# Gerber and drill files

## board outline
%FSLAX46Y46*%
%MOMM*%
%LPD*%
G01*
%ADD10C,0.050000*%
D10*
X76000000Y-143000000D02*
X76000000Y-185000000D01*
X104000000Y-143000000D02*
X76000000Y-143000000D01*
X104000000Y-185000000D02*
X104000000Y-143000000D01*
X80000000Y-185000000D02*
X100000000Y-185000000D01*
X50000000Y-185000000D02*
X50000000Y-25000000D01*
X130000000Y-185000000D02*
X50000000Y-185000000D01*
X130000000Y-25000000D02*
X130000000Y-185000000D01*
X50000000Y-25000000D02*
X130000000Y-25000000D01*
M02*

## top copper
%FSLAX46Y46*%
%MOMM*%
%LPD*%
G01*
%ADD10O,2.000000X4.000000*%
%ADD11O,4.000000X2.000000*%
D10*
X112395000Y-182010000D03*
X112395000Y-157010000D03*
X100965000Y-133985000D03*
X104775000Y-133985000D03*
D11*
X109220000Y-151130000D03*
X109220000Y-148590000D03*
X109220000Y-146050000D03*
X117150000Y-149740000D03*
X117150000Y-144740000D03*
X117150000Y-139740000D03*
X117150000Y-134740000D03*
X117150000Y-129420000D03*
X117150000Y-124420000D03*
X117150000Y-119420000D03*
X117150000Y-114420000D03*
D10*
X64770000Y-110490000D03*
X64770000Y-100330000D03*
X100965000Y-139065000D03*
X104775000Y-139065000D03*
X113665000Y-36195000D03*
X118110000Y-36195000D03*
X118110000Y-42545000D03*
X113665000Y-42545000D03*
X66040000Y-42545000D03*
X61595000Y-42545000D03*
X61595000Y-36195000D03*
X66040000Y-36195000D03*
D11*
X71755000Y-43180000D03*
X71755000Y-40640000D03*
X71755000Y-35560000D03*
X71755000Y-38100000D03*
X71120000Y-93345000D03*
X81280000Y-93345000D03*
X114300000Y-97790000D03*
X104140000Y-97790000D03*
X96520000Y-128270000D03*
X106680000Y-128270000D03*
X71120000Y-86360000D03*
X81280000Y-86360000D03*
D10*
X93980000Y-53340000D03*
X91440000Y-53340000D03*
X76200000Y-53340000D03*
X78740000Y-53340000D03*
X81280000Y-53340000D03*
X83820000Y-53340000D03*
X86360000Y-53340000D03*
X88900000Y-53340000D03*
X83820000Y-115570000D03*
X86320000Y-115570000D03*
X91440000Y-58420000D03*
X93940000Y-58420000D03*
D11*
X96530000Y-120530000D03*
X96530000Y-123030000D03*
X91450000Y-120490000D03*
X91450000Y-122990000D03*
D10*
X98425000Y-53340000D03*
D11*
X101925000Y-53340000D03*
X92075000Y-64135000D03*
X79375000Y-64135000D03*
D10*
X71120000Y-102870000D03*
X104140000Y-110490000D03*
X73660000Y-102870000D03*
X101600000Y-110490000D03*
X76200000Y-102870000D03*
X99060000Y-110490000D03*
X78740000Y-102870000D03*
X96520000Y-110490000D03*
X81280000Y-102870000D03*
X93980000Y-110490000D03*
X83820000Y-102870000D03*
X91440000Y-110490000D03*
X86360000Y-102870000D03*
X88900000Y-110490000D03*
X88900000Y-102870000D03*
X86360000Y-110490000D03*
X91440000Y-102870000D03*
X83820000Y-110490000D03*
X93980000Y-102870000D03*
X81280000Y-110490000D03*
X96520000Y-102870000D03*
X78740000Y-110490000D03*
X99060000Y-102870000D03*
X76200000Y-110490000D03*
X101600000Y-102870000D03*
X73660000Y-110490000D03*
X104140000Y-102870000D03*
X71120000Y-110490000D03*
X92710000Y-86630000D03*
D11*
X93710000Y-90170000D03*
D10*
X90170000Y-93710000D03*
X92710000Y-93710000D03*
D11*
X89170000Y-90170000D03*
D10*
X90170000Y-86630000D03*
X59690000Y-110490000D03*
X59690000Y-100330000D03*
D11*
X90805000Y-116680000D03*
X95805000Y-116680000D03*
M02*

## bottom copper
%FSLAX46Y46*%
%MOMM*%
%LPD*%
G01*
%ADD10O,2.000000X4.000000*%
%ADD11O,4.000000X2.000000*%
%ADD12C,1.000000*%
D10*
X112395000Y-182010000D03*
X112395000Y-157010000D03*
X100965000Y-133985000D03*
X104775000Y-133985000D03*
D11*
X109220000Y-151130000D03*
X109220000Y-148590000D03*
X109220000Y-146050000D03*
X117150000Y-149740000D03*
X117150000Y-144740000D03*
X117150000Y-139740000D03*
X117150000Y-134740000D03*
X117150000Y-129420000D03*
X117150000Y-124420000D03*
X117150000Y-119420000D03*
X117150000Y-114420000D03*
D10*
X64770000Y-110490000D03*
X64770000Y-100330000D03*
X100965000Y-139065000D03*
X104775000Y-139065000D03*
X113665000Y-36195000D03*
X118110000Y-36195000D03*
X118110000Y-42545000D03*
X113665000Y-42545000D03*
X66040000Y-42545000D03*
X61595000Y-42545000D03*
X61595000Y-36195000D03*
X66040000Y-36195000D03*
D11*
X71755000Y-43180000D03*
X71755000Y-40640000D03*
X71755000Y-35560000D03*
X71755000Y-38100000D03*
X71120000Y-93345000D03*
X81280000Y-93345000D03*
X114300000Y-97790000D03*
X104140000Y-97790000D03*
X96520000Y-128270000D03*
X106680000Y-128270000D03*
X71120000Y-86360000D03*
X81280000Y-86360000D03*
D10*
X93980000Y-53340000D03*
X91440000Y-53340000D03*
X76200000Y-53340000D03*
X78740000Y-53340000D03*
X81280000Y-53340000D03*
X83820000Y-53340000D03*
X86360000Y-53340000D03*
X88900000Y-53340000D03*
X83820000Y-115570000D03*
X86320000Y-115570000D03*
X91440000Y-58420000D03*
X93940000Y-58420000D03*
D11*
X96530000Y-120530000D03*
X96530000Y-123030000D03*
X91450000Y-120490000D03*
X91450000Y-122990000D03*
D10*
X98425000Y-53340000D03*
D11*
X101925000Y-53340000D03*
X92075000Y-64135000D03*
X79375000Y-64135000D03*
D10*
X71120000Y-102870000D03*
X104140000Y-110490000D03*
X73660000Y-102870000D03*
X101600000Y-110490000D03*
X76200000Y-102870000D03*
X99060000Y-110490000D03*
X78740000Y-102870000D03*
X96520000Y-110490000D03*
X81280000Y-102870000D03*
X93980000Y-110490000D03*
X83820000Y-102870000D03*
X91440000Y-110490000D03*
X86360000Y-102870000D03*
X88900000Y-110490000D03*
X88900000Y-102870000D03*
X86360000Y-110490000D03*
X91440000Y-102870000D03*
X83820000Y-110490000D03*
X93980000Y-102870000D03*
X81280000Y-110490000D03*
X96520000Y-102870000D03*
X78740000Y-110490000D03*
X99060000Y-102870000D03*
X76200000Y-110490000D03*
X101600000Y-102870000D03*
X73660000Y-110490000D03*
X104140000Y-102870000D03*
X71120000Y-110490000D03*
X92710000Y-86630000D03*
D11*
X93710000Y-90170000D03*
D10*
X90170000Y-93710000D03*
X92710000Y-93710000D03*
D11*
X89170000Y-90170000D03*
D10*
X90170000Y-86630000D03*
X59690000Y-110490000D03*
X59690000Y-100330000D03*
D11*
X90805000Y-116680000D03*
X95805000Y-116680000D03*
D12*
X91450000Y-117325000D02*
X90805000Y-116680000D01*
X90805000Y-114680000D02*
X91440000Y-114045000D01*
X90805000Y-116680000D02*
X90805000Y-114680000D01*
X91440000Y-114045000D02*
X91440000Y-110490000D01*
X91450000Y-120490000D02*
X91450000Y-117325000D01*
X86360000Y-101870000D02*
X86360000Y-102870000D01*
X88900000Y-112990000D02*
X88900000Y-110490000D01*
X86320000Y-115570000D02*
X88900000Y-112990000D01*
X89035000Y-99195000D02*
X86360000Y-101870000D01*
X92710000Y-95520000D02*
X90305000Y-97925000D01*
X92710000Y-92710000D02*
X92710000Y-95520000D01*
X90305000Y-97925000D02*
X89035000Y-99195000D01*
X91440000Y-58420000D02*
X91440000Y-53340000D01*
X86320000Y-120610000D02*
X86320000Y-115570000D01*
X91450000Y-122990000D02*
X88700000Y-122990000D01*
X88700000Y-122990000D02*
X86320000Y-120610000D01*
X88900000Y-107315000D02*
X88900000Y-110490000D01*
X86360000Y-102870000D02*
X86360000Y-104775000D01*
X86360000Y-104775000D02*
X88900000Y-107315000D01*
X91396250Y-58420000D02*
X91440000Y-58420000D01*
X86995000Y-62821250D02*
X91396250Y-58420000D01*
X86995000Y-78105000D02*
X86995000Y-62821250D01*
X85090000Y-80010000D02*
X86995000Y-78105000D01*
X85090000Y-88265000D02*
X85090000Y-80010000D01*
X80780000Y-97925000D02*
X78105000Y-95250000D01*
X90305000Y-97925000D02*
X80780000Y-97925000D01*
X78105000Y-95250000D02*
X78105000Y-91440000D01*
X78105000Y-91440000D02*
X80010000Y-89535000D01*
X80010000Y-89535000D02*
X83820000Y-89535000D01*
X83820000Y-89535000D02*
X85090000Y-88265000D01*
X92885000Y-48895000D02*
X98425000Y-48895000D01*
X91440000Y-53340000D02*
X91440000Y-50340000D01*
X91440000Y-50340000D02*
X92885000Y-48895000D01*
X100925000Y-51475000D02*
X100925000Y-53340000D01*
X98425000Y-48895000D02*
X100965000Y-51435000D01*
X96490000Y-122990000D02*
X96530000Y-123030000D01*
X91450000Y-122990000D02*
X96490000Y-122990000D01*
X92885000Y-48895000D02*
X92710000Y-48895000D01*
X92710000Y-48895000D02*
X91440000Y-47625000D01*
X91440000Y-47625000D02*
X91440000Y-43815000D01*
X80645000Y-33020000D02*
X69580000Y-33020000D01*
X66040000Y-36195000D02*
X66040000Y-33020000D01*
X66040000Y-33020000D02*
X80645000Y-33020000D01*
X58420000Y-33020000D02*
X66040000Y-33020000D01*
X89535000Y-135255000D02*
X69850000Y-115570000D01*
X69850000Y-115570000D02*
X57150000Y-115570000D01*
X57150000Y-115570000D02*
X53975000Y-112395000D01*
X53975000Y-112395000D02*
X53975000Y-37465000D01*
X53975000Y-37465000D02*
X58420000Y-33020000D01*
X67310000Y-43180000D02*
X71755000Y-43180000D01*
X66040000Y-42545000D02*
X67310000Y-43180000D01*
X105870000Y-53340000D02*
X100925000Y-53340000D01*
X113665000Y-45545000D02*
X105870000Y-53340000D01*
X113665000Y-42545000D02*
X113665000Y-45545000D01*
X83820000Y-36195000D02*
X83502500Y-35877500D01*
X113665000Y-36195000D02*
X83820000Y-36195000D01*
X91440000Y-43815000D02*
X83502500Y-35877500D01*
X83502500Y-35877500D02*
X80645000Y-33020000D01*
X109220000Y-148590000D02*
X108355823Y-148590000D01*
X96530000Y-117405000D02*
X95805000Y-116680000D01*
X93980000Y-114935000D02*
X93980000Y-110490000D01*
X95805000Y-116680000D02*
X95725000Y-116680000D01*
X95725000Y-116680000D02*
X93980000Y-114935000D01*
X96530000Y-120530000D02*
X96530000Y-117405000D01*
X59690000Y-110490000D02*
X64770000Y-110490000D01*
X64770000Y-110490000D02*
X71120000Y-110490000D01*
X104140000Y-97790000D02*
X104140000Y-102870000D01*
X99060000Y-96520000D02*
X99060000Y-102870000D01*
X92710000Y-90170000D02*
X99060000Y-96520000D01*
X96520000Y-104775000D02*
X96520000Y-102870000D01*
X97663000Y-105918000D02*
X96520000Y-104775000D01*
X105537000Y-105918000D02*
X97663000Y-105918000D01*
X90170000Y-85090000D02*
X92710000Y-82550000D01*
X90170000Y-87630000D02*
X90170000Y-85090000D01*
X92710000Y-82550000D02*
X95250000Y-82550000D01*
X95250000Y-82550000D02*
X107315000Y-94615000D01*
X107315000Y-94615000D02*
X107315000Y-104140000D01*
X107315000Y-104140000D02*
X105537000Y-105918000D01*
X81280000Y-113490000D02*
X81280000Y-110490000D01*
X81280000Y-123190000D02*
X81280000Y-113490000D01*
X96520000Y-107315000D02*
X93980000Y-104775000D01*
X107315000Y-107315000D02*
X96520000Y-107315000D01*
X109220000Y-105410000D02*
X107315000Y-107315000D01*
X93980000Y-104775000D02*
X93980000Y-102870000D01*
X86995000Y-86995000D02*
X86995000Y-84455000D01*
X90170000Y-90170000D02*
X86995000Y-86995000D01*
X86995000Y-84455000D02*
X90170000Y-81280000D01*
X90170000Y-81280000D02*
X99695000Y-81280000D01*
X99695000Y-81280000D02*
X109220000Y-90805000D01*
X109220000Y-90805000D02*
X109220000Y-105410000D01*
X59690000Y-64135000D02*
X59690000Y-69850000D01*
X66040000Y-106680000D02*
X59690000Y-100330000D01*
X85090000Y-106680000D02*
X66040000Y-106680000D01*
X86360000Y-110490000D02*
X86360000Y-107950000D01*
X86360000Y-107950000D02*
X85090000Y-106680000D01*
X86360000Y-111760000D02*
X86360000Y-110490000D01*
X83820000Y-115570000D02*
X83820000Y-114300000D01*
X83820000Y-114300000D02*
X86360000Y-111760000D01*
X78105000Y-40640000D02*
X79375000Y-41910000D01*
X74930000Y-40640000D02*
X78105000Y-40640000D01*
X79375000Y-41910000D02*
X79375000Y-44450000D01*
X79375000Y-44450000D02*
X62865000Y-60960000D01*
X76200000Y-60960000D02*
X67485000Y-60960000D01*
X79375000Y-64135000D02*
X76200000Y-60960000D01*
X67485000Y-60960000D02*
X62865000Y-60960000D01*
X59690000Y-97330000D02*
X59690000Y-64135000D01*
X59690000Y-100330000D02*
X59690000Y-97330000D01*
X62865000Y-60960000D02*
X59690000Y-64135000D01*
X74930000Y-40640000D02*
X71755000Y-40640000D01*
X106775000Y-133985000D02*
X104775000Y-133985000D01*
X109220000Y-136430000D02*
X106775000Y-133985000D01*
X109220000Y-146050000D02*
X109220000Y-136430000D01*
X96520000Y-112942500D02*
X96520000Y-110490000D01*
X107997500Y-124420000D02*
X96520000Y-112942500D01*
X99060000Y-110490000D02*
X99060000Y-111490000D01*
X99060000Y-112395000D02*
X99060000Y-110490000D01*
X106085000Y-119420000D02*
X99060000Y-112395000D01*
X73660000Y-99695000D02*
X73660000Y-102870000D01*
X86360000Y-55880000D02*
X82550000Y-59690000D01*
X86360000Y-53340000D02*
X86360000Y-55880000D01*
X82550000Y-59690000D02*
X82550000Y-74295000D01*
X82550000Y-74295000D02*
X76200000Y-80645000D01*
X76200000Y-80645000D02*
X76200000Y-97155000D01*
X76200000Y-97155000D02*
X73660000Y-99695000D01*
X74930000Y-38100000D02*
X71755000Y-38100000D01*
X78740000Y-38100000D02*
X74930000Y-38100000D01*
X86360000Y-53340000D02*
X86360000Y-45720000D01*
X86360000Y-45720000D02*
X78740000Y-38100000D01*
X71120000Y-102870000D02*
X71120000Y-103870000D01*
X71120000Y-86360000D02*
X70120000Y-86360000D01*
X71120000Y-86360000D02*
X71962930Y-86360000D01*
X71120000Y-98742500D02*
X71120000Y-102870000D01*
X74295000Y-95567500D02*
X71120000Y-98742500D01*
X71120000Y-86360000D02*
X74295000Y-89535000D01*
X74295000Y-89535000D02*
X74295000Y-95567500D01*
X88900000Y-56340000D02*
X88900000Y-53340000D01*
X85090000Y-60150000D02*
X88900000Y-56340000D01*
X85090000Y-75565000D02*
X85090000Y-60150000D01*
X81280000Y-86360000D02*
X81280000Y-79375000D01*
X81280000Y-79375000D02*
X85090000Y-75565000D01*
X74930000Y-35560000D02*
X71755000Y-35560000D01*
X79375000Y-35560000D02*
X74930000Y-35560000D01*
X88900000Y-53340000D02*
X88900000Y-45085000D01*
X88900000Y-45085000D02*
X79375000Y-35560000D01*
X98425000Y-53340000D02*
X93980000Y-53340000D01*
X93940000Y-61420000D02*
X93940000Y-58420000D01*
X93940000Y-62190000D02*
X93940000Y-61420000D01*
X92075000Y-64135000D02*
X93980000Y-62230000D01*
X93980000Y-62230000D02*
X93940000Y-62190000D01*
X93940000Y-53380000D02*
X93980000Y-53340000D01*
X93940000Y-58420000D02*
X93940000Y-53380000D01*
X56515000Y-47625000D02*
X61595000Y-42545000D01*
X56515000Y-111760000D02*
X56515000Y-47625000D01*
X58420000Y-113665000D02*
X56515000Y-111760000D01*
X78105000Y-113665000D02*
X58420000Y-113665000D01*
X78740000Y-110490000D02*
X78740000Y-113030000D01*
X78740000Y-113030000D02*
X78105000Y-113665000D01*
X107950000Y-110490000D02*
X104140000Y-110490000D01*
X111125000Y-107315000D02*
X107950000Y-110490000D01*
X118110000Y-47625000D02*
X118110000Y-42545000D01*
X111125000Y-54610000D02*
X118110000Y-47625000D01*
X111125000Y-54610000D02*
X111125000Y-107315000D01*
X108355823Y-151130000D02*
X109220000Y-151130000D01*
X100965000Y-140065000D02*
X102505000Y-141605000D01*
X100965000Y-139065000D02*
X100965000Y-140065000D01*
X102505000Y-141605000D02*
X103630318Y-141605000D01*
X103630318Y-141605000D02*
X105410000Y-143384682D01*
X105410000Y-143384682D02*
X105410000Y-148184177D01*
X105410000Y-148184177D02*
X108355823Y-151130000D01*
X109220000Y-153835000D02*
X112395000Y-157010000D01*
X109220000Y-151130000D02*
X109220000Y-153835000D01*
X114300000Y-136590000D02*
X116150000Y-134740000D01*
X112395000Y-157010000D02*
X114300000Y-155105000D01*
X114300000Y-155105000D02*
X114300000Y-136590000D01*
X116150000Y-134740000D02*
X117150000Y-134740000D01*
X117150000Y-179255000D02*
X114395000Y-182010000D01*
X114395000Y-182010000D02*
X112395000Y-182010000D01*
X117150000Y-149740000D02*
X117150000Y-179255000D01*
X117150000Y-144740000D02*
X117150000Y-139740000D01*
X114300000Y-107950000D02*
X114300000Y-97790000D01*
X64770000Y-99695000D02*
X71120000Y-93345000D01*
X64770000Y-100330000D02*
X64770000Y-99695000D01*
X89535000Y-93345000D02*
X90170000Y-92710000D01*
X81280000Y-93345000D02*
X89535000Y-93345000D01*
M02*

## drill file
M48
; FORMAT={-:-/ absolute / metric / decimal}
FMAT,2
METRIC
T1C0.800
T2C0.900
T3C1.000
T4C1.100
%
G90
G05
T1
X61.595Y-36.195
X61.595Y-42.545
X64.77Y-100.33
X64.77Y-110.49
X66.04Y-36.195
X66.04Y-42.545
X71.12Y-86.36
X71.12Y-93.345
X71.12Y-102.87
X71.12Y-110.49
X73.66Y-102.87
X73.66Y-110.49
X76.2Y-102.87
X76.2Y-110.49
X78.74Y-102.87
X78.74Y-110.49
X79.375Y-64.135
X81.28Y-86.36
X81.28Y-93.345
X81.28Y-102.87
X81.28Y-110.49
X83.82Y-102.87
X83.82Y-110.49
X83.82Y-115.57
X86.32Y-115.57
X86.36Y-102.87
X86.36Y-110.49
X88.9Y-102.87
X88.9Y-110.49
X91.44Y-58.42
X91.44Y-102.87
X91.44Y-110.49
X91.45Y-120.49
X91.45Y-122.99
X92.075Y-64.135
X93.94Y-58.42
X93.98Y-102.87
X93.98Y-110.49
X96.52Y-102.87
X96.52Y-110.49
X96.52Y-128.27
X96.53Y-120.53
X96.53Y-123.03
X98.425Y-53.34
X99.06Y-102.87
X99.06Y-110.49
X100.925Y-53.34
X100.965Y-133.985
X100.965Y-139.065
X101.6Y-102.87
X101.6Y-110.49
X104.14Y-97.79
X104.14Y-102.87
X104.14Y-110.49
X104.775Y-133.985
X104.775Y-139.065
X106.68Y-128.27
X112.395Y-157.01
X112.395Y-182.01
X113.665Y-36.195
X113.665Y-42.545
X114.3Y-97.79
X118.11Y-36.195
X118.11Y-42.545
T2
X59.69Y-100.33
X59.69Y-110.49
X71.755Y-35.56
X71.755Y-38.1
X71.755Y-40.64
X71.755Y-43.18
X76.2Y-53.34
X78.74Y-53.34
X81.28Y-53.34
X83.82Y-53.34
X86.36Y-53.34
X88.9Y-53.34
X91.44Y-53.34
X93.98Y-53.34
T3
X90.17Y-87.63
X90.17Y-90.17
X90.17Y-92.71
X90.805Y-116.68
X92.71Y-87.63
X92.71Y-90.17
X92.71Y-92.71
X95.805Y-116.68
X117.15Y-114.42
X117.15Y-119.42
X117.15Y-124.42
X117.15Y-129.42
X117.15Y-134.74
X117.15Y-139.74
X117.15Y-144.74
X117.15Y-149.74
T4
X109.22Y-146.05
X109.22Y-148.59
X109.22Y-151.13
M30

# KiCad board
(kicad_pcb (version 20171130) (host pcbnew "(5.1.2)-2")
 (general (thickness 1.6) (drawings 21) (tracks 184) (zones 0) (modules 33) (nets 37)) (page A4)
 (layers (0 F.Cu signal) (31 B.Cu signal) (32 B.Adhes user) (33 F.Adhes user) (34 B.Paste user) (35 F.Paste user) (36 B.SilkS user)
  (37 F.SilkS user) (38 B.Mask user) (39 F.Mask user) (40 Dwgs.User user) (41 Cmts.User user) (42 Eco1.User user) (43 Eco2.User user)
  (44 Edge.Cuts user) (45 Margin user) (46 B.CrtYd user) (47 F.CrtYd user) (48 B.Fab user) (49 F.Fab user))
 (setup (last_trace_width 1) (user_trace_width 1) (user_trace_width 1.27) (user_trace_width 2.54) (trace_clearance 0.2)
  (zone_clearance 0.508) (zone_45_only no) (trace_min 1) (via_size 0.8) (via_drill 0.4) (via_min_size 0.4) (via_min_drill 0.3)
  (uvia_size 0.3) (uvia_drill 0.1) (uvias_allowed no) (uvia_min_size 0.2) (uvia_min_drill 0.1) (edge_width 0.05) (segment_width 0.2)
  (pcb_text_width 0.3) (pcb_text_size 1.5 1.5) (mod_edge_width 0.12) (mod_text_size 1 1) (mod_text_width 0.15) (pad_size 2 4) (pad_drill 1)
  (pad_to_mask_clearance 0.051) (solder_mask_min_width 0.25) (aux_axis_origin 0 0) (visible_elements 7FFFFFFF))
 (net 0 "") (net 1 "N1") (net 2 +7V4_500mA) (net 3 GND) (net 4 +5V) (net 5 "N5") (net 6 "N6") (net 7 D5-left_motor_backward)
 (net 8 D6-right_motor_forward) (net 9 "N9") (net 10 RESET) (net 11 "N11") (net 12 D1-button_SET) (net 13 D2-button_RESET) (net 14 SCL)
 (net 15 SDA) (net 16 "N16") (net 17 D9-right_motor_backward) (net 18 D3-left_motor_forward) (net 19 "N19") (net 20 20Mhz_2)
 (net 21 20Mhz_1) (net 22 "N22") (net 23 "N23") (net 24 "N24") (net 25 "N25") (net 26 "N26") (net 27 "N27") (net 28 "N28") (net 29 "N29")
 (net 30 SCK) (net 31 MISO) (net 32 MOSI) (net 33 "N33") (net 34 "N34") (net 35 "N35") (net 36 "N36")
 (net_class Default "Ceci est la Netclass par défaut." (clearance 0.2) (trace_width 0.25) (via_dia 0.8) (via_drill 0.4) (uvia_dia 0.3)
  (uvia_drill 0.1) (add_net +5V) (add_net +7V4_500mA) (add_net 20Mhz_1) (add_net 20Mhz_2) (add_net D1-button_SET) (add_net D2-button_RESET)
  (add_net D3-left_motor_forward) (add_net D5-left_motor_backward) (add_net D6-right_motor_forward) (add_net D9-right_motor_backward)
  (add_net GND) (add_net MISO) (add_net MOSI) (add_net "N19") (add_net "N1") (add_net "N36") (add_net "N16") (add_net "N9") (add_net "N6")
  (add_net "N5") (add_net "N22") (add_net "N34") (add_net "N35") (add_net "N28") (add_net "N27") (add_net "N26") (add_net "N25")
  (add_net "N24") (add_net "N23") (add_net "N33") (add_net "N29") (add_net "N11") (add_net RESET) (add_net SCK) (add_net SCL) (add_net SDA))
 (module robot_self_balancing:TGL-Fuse (layer F.Cu) (at 121.285 168.91 270)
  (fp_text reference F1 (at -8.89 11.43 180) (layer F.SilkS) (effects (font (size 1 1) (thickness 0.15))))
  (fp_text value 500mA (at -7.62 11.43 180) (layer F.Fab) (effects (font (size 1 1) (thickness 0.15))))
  (pad 2 thru_hole oval (at 13.1 8.89 270) (size 4 2) (drill 0.8) (layers *.Cu *.Mask) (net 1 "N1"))
  (pad 1 thru_hole oval (at -11.9 8.89 270) (size 4 2) (drill 0.8) (layers *.Cu *.Mask) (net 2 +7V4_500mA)))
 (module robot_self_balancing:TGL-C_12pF (layer F.Cu) (at 104.14 133.985 180)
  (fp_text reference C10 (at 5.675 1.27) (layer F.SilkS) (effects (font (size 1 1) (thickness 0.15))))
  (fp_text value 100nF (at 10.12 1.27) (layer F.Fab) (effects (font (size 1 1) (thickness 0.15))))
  (pad 2 thru_hole oval (at 3.175 0 180) (size 2 4) (drill 0.8) (layers *.Cu *.Mask) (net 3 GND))
  (pad 1 thru_hole oval (at -0.635 0 180) (size 2 4) (drill 0.8) (layers *.Cu *.Mask) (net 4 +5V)))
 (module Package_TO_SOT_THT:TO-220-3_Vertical (layer F.Cu) (at 109.22 151.13 90)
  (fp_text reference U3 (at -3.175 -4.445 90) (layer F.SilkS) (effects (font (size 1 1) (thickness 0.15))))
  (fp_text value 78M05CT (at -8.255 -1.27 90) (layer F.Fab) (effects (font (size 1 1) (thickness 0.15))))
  (pad 1 thru_hole oval (at 0 0 90) (size 2 4) (drill 1.1) (layers *.Cu *.Mask) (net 2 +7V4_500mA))
  (pad 2 thru_hole oval (at 2.54 0 90) (size 2 4) (drill 1.1) (layers *.Cu *.Mask) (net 3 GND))
  (pad 3 thru_hole oval (at 5.08 0 90) (size 2 4) (drill 1.1) (layers *.Cu *.Mask) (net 4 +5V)))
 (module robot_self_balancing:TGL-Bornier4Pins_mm (layer F.Cu) (at 120.65 142.24 270)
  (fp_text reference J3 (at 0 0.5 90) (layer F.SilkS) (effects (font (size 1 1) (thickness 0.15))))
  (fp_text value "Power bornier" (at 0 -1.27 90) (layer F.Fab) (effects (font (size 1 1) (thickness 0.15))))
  (pad 5 thru_hole oval (at 7.5 3.5 90) (size 2 4) (drill 1) (layers *.Cu *.Mask) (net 1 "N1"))
  (pad 7 thru_hole oval (at 2.5 3.5 270) (size 2 4) (drill 1) (layers *.Cu *.Mask) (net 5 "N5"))
  (pad 6 thru_hole oval (at -2.5 3.5 270) (size 2 4) (drill 1) (layers *.Cu *.Mask) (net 5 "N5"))
  (pad 8 thru_hole oval (at -7.5 3.5 270) (size 2 4) (drill 1) (layers *.Cu *.Mask) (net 2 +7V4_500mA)))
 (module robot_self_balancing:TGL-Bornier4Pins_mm (layer F.Cu) (at 120.65 121.92 270)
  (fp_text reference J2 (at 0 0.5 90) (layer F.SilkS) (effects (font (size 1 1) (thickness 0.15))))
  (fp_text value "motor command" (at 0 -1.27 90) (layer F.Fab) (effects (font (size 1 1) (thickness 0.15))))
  (pad 8 thru_hole oval (at 7.5 3.5 90) (size 2 4) (drill 1) (layers *.Cu *.Mask) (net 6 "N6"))
  (pad 7 thru_hole oval (at 2.5 3.5 270) (size 2 4) (drill 1) (layers *.Cu *.Mask) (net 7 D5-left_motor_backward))
  (pad 6 thru_hole oval (at -2.5 3.5 270) (size 2 4) (drill 1) (layers *.Cu *.Mask) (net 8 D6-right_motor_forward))
  (pad 5 thru_hole oval (at -7.5 3.5 270) (size 2 4) (drill 1) (layers *.Cu *.Mask) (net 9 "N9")))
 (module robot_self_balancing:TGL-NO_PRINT (layer F.Cu) (at 168.22 120.57)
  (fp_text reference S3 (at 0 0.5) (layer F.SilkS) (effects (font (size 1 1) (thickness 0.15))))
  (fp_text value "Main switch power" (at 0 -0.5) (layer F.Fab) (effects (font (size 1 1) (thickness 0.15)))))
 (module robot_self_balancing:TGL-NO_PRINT (layer F.Cu) (at 168.22 113.03)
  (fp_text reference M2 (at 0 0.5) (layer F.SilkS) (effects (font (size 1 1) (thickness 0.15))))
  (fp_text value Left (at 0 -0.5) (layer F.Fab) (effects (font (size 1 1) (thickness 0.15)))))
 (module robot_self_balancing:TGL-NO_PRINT (layer F.Cu) (at 162.1 120.57)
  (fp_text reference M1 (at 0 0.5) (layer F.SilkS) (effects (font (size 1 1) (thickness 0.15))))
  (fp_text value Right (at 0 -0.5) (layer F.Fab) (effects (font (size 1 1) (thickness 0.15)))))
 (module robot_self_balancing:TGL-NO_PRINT (layer F.Cu) (at 155.98 120.57)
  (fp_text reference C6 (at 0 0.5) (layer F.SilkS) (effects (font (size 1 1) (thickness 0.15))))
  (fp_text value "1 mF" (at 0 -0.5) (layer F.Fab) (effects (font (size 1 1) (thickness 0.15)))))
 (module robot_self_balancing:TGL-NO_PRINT (layer F.Cu) (at 162.1 113.03)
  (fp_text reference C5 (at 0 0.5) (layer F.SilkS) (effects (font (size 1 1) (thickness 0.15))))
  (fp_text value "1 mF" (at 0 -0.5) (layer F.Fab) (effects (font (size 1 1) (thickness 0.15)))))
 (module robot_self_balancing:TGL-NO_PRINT (layer F.Cu) (at 155.98 113.03)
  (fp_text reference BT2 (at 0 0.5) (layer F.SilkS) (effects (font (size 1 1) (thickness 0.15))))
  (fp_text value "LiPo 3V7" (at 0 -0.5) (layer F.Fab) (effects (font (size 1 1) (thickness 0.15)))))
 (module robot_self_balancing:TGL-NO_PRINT (layer F.Cu) (at 149.86 120.57)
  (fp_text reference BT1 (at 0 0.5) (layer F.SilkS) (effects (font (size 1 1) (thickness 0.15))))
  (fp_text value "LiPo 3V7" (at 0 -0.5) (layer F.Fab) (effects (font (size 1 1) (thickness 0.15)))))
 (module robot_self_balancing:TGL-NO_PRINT (layer F.Cu) (at 149.86 113.03)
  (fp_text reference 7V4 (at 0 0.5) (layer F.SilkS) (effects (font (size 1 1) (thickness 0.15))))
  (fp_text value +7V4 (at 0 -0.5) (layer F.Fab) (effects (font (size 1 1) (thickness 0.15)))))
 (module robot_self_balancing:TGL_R (layer F.Cu) (at 64.77 100.33 270)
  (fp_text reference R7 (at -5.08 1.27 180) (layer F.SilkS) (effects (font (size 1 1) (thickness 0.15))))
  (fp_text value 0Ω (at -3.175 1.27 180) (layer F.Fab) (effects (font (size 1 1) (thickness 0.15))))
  (pad 2 thru_hole oval (at 10.16 0 270) (size 4 2) (drill 0.8) (layers *.Cu *.Mask) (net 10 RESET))
  (pad 1 thru_hole oval (at 0 0 270) (size 4 2) (drill 0.8) (layers *.Cu *.Mask) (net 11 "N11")))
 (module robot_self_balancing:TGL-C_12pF (layer F.Cu) (at 104.14 139.065 180)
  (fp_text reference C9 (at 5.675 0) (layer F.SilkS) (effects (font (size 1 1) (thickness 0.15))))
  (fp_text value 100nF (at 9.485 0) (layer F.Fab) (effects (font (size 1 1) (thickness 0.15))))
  (pad 2 thru_hole oval (at 3.175 0 180) (size 2 4) (drill 0.8) (layers *.Cu *.Mask) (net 2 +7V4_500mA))
  (pad 1 thru_hole oval (at -0.635 0 180) (size 2 4) (drill 0.8) (layers *.Cu *.Mask) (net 3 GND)))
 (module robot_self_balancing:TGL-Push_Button (layer F.Cu) (at 111.125 39.37 90)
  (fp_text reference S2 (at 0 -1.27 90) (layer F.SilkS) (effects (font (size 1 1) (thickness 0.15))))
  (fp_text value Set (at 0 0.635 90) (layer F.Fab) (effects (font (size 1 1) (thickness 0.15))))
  (pad 1 thru_hole oval (at 3.175 2.54 90) (size 4 2) (drill 0.8) (layers *.Cu *.Mask) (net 3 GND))
  (pad 2 thru_hole oval (at 3.175 6.985 90) (size 4 2) (drill 0.8) (layers *.Cu *.Mask) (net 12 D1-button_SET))
  (pad 2 thru_hole oval (at -3.175 6.985 90) (size 4 2) (drill 0.8) (layers *.Cu *.Mask) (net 12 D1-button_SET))
  (pad 1 thru_hole oval (at -3.175 2.54 90) (size 4 2) (drill 0.8) (layers *.Cu *.Mask) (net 3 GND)))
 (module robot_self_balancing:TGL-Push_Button (layer F.Cu) (at 68.58 39.37 270)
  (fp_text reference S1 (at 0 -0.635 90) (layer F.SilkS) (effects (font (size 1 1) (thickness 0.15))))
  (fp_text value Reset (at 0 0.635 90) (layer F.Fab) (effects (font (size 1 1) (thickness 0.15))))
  (pad 1 thru_hole oval (at 3.175 2.54 270) (size 4 2) (drill 0.8) (layers *.Cu *.Mask) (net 3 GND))
  (pad 2 thru_hole oval (at 3.175 6.985 270) (size 4 2) (drill 0.8) (layers *.Cu *.Mask) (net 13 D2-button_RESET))
  (pad 2 thru_hole oval (at -3.175 6.985 270) (size 4 2) (drill 0.8) (layers *.Cu *.Mask) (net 13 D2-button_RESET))
  (pad 1 thru_hole oval (at -3.175 2.54 270) (size 4 2) (drill 0.8) (layers *.Cu *.Mask) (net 3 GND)))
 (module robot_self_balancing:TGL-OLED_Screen (layer F.Cu) (at 67.945 39.37 90)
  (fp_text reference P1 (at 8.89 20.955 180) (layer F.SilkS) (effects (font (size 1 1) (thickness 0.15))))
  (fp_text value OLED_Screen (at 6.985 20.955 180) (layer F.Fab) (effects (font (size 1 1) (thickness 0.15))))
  (pad 1 thru_hole oval (at -3.81 3.81 90) (size 2 4) (drill 0.9) (layers *.Cu *.Mask) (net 3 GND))
  (pad 2 thru_hole oval (at -1.27 3.81 90) (size 2 4) (drill 0.9) (layers *.Cu *.Mask) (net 4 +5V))
  (pad 4 thru_hole oval (at 3.81 3.81 90) (size 2 4) (drill 0.9) (layers *.Cu *.Mask) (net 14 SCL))
  (pad 3 thru_hole oval (at 1.27 3.81 90) (size 2 4) (drill 0.9) (layers *.Cu *.Mask) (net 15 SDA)))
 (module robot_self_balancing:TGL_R (layer F.Cu) (at 81.28 93.345 180)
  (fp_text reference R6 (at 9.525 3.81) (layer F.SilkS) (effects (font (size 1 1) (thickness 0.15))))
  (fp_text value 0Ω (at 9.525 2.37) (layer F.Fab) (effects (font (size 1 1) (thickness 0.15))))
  (pad 2 thru_hole oval (at 10.16 0 180) (size 4 2) (drill 0.8) (layers *.Cu *.Mask) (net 11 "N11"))
  (pad 1 thru_hole oval (at 0 0 180) (size 4 2) (drill 0.8) (layers *.Cu *.Mask) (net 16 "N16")))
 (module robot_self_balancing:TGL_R (layer F.Cu) (at 104.14 97.79)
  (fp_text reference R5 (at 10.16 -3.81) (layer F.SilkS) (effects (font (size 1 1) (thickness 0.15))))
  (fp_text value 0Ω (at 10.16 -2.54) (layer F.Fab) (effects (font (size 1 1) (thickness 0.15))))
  (pad 2 thru_hole oval (at 10.16 0) (size 4 2) (drill 0.8) (layers *.Cu *.Mask) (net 9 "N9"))
  (pad 1 thru_hole oval (at 0 0) (size 4 2) (drill 0.8) (layers *.Cu *.Mask) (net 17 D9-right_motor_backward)))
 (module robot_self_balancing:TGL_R (layer F.Cu) (at 106.68 128.27 180)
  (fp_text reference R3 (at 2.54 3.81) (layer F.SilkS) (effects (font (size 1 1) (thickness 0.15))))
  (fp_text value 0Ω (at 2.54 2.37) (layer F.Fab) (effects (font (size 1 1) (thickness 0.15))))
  (pad 2 thru_hole oval (at 10.16 0 180) (size 4 2) (drill 0.8) (layers *.Cu *.Mask) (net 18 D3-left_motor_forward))
  (pad 1 thru_hole oval (at 0 0 180) (size 4 2) (drill 0.8) (layers *.Cu *.Mask) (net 6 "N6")))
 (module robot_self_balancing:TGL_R (layer F.Cu) (at 81.28 86.36 180)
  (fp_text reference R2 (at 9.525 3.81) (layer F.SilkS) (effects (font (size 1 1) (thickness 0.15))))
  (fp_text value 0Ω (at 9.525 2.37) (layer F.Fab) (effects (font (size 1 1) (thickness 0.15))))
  (pad 2 thru_hole oval (at 10.16 0 180) (size 4 2) (drill 0.8) (layers *.Cu *.Mask) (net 14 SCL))
  (pad 1 thru_hole oval (at 0 0 180) (size 4 2) (drill 0.8) (layers *.Cu *.Mask) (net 14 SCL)))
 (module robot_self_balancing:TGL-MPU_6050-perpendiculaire (layer F.Cu) (at 85.09 57.15 180)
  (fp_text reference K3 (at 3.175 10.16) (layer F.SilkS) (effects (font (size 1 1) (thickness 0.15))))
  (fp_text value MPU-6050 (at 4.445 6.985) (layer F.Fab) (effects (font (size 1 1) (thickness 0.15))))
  (pad 13 thru_hole oval (at -8.89 3.81 180) (size 2 4) (drill 0.9) (layers *.Cu *.Mask) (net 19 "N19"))
  (pad 18 thru_hole oval (at -6.35 3.81 180) (size 2 4) (drill 0.9) (layers *.Cu *.Mask) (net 3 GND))
  (pad "" thru_hole oval (at 8.89 3.81 180) (size 2 4) (drill 0.9) (layers *.Cu *.Mask))
  (pad "" thru_hole oval (at 6.35 3.81 180) (size 2 4) (drill 0.9) (layers *.Cu *.Mask))
  (pad "" thru_hole oval (at 3.81 3.81 180) (size 2 4) (drill 0.9) (layers *.Cu *.Mask))
  (pad "" thru_hole oval (at 1.27 3.81 180) (size 2 4) (drill 0.9) (layers *.Cu *.Mask))
  (pad 24 thru_hole oval (at -1.27 3.81 180) (size 2 4) (drill 0.9) (layers *.Cu *.Mask) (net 15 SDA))
  (pad 23 thru_hole oval (at -3.81 3.81 180) (size 2 4) (drill 0.9) (layers *.Cu *.Mask) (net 14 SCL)))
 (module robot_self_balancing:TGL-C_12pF (layer F.Cu) (at 86.32 115.57 180)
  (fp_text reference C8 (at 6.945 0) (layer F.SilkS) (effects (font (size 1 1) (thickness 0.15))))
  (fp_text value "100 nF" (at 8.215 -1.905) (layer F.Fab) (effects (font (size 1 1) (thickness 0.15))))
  (pad 2 thru_hole oval (at 2.5 0 180) (size 2 4) (drill 0.8) (layers *.Cu *.Mask) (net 4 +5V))
  (pad 1 thru_hole oval (at 0 0 180) (size 2 4) (drill 0.8) (layers *.Cu *.Mask) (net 3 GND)))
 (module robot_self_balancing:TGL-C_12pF (layer F.Cu) (at 93.94 58.42 180)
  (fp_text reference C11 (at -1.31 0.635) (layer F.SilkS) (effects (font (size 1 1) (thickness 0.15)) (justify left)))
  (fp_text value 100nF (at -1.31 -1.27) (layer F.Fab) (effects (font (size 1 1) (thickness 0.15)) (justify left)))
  (pad 2 thru_hole oval (at 2.5 0 180) (size 2 4) (drill 0.8) (layers *.Cu *.Mask) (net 3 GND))
  (pad 1 thru_hole oval (at 0 0 180) (size 2 4) (drill 0.8) (layers *.Cu *.Mask) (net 19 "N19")))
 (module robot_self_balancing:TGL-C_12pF (layer F.Cu) (at 96.53 120.53 270)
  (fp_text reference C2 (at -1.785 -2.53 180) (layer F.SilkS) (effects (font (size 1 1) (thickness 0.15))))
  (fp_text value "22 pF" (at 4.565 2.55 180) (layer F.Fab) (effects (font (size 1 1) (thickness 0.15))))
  (pad 1 thru_hole oval (at 0 0 270) (size 2 4) (drill 0.8) (layers *.Cu *.Mask) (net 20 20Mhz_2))
  (pad 2 thru_hole oval (at 2.5 0 270) (size 2 4) (drill 0.8) (layers *.Cu *.Mask) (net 3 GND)))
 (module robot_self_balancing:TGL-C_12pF (layer F.Cu) (at 91.45 120.49 270)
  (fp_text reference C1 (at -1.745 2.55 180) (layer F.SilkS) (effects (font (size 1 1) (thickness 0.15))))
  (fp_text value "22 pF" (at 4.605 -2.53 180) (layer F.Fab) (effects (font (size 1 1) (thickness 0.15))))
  (pad 1 thru_hole oval (at 0 0 270) (size 2 4) (drill 0.8) (layers *.Cu *.Mask) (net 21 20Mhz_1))
  (pad 2 thru_hole oval (at 2.5 0 270) (size 2 4) (drill 0.8) (layers *.Cu *.Mask) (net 3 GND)))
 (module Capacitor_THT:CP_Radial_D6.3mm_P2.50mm (layer F.Cu) (at 98.425 53.34)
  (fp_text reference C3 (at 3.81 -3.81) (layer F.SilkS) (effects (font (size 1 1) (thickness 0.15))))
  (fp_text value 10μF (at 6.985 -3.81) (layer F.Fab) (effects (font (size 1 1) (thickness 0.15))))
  (pad 1 thru_hole oval (at 0 0) (size 2 4) (drill 0.8) (layers *.Cu *.Mask) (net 19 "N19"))
  (pad 2 thru_hole oval (at 2.5 0) (size 4 2) (drill 0.8 (offset 1 0)) (layers *.Cu *.Mask) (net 3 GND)))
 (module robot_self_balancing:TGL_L (layer F.Cu) (at 92.075 64.135 180)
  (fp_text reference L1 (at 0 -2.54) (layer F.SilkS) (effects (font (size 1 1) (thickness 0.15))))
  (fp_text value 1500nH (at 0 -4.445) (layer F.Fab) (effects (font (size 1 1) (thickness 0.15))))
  (pad 1 thru_hole oval (at 0 0 180) (size 4 2) (drill 0.8) (layers *.Cu *.Mask) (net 19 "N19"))
  (pad 2 thru_hole oval (at 12.7 0 180) (size 4 2) (drill 0.8) (layers *.Cu *.Mask) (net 4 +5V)))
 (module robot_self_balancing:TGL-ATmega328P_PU (layer F.Cu) (at 71.12 110.49 90)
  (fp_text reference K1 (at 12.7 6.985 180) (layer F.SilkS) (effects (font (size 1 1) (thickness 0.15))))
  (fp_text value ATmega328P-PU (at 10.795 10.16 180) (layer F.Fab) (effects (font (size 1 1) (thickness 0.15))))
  (pad 28 thru_hole oval (at 7.62 0 90) (size 4 2) (drill 0.8) (layers *.Cu *.Mask) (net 14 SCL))
  (pad 14 thru_hole oval (at 0 33.02 90) (size 4 2) (drill 0.8) (layers *.Cu *.Mask) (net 12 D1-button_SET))
  (pad 27 thru_hole oval (at 7.62 2.54 90) (size 4 2) (drill 0.8) (layers *.Cu *.Mask) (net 15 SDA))
  (pad 13 thru_hole oval (at 0 30.48 90) (size 4 2) (drill 0.8) (layers *.Cu *.Mask) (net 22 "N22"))
  (pad 26 thru_hole oval (at 7.62 5.08 90) (size 4 2) (drill 0.8) (layers *.Cu *.Mask) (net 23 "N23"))
  (pad 12 thru_hole oval (at 0 27.94 90) (size 4 2) (drill 0.8) (layers *.Cu *.Mask) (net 8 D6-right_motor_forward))
  (pad 25 thru_hole oval (at 7.62 7.62 90) (size 4 2) (drill 0.8) (layers *.Cu *.Mask) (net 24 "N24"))
  (pad 11 thru_hole oval (at 0 25.4 90) (size 4 2) (drill 0.8) (layers *.Cu *.Mask) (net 7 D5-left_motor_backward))
  (pad 24 thru_hole oval (at 7.62 10.16 90) (size 4 2) (drill 0.8) (layers *.Cu *.Mask) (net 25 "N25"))
  (pad 10 thru_hole oval (at 0 22.86 90) (size 4 2) (drill 0.8) (layers *.Cu *.Mask) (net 20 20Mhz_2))
  (pad 23 thru_hole oval (at 7.62 12.7 90) (size 4 2) (drill 0.8) (layers *.Cu *.Mask) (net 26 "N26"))
  (pad 9 thru_hole oval (at 0 20.32 90) (size 4 2) (drill 0.8) (layers *.Cu *.Mask) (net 21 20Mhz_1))
  (pad 22 thru_hole oval (at 7.62 15.24 90) (size 4 2) (drill 0.8) (layers *.Cu *.Mask) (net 3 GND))
  (pad 8 thru_hole oval (at 0 17.78 90) (size 4 2) (drill 0.8) (layers *.Cu *.Mask) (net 3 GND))
  (pad 21 thru_hole oval (at 7.62 17.78 90) (size 4 2) (drill 0.8) (layers *.Cu *.Mask) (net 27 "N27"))
  (pad 7 thru_hole oval (at 0 15.24 90) (size 4 2) (drill 0.8) (layers *.Cu *.Mask) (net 4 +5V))
  (pad 20 thru_hole oval (at 7.62 20.32 90) (size 4 2) (drill 0.8) (layers *.Cu *.Mask) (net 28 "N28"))
  (pad 6 thru_hole oval (at 0 12.7 90) (size 4 2) (drill 0.8) (layers *.Cu *.Mask) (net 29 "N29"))
  (pad 19 thru_hole oval (at 7.62 22.86 90) (size 4 2) (drill 0.8) (layers *.Cu *.Mask) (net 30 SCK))
  (pad 5 thru_hole oval (at 0 10.16 90) (size 4 2) (drill 0.8) (layers *.Cu *.Mask) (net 18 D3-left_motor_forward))
  (pad 18 thru_hole oval (at 7.62 25.4 90) (size 4 2) (drill 0.8) (layers *.Cu *.Mask) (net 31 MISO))
  (pad 4 thru_hole oval (at 0 7.62 90) (size 4 2) (drill 0.8) (layers *.Cu *.Mask) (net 13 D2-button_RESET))
  (pad 17 thru_hole oval (at 7.62 27.94 90) (size 4 2) (drill 0.8) (layers *.Cu *.Mask) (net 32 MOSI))
  (pad 3 thru_hole oval (at 0 5.08 90) (size 4 2) (drill 0.8) (layers *.Cu *.Mask) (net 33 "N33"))
  (pad 16 thru_hole oval (at 7.62 30.48 90) (size 4 2) (drill 0.8) (layers *.Cu *.Mask) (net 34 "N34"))
  (pad 2 thru_hole oval (at 0 2.54 90) (size 4 2) (drill 0.8) (layers *.Cu *.Mask) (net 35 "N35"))
  (pad 15 thru_hole oval (at 7.62 33.02 90) (size 4 2) (drill 0.8) (layers *.Cu *.Mask) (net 17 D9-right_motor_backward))
  (pad 1 thru_hole oval (at 0 0 90) (size 4 2) (drill 0.8) (layers *.Cu *.Mask) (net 10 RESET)))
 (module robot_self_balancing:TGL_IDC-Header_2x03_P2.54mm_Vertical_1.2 (layer F.Cu) (at 90.17 87.63)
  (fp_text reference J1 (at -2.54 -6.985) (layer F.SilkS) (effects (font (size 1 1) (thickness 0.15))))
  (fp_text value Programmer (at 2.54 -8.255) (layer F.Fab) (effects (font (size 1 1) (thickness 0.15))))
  (pad 2 thru_hole oval (at 2.54 0) (size 2 4) (drill 1 (offset 0 -1)) (layers *.Cu *.Mask) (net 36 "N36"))
  (pad 4 thru_hole oval (at 2.54 2.54) (size 4 2) (drill 1 (offset 1 0)) (layers *.Cu *.Mask) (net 32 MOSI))
  (pad 5 thru_hole oval (at 0 5.08) (size 2 4) (drill 1 (offset 0 1)) (layers *.Cu *.Mask) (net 16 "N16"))
  (pad 6 thru_hole oval (at 2.54 5.08) (size 2 4) (drill 1 (offset 0 1)) (layers *.Cu *.Mask) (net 3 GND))
  (pad 3 thru_hole oval (at 0 2.54) (size 4 2) (drill 1 (offset -1 0)) (layers *.Cu *.Mask) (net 30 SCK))
  (pad 1 thru_hole oval (at 0 0) (size 2 4) (drill 1 (offset 0 -1)) (layers *.Cu *.Mask) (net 31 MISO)))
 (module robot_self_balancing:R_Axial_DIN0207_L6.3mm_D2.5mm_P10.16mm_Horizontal (layer F.Cu) (at 59.69 100.33 270)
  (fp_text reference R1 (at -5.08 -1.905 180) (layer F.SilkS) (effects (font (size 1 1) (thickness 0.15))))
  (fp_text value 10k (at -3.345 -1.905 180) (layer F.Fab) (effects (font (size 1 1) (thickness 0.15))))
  (pad 2 thru_hole oval (at 10.16 0 270) (size 4 2) (drill 0.9) (layers *.Cu *.Mask) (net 10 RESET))
  (pad 1 thru_hole oval (at 0 0 270) (size 4 2) (drill 0.9) (layers *.Cu *.Mask) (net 4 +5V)))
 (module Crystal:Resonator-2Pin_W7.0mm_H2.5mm (layer F.Cu) (at 90.805 116.68)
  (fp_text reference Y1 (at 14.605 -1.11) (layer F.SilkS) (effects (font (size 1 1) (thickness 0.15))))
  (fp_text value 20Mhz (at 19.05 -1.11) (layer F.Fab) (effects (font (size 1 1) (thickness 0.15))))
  (pad 1 thru_hole oval (at 0 0) (size 4 2) (drill 1) (layers *.Cu *.Mask) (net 21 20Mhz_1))
  (pad 2 thru_hole oval (at 5 0) (size 4 2) (drill 1) (layers *.Cu *.Mask) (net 20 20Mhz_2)))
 (gr_line (start 76 143) (end 76 185) (layer Edge.Cuts) (width 0.05))
 (gr_line (start 104 143) (end 76 143) (layer Edge.Cuts) (width 0.05))
 (gr_line (start 104 185) (end 104 143) (layer Edge.Cuts) (width 0.05))
 (gr_line (start 80 185) (end 100 185) (layer Edge.Cuts) (width 0.05))
 (gr_line (start 50 185) (end 50 25) (layer Edge.Cuts) (width 0.05))
 (gr_line (start 130 185) (end 50 185) (layer Edge.Cuts) (width 0.05))
 (gr_line (start 130 25) (end 130 185) (layer Edge.Cuts) (width 0.05))
 (gr_line (start 50 25) (end 130 25) (layer Edge.Cuts) (width 0.05))
 (segment (start 91.45 117.325) (end 90.805 116.68) (width 1) (layer B.Cu) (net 21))
 (segment (start 90.805 114.68) (end 91.44 114.045) (width 1) (layer B.Cu) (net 21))
 (segment (start 90.805 116.68) (end 90.805 114.68) (width 1) (layer B.Cu) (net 21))
 (segment (start 91.44 114.045) (end 91.44 110.49) (width 1) (layer B.Cu) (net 21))
 (segment (start 91.45 120.49) (end 91.45 117.325) (width 1) (layer B.Cu) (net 21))
 (segment (start 86.36 101.87) (end 86.36 102.87) (width 1) (layer B.Cu) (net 3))
 (segment (start 88.9 112.99) (end 88.9 110.49) (width 1) (layer B.Cu) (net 3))
 (segment (start 86.32 115.57) (end 88.9 112.99) (width 1) (layer B.Cu) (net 3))
 (segment (start 89.035 99.195) (end 86.36 101.87) (width 1) (layer B.Cu) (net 3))
 (segment (start 92.71 95.52) (end 90.305 97.925) (width 1) (layer B.Cu) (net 3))
 (segment (start 92.71 92.71) (end 92.71 95.52) (width 1) (layer B.Cu) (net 3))
 (segment (start 90.305 97.925) (end 89.035 99.195) (width 1) (layer B.Cu) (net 3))
 (segment (start 91.44 58.42) (end 91.44 53.34) (width 1) (layer B.Cu) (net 3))
 (segment (start 86.32 120.61) (end 86.32 115.57) (width 1) (layer B.Cu) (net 3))
 (segment (start 91.45 122.99) (end 88.7 122.99) (width 1) (layer B.Cu) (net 3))
 (segment (start 88.7 122.99) (end 86.32 120.61) (width 1) (layer B.Cu) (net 3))
 (segment (start 88.9 107.315) (end 88.9 110.49) (width 1) (layer B.Cu) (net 3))
 (segment (start 86.36 102.87) (end 86.36 104.775) (width 1) (layer B.Cu) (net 3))
 (segment (start 86.36 104.775) (end 88.9 107.315) (width 1) (layer B.Cu) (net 3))
 (segment (start 91.39625 58.42) (end 91.44 58.42) (width 1) (layer B.Cu) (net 3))
 (segment (start 86.995 62.82125) (end 91.39625 58.42) (width 1) (layer B.Cu) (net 3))
 (segment (start 86.995 78.105) (end 86.995 62.82125) (width 1) (layer B.Cu) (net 3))
 (segment (start 85.09 80.01) (end 86.995 78.105) (width 1) (layer B.Cu) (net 3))
 (segment (start 85.09 88.265) (end 85.09 80.01) (width 1) (layer B.Cu) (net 3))
 (segment (start 80.78 97.925) (end 78.105 95.25) (width 1) (layer B.Cu) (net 3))
 (segment (start 90.305 97.925) (end 80.78 97.925) (width 1) (layer B.Cu) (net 3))
 (segment (start 78.105 95.25) (end 78.105 91.44) (width 1) (layer B.Cu) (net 3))
 (segment (start 78.105 91.44) (end 80.01 89.535) (width 1) (layer B.Cu) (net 3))
 (segment (start 80.01 89.535) (end 83.82 89.535) (width 1) (layer B.Cu) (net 3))
 (segment (start 83.82 89.535) (end 85.09 88.265) (width 1) (layer B.Cu) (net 3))
 (segment (start 92.885 48.895) (end 98.425 48.895) (width 1) (layer B.Cu) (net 3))
 (segment (start 91.44 53.34) (end 91.44 50.34) (width 1) (layer B.Cu) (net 3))
 (segment (start 91.44 50.34) (end 92.885 48.895) (width 1) (layer B.Cu) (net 3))
 (segment (start 100.925 51.475) (end 100.925 53.34) (width 1) (layer B.Cu) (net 3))
 (segment (start 98.425 48.895) (end 100.965 51.435) (width 1) (layer B.Cu) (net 3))
 (segment (start 96.49 122.99) (end 96.53 123.03) (width 1) (layer B.Cu) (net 3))
 (segment (start 91.45 122.99) (end 96.49 122.99) (width 1) (layer B.Cu) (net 3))
 (segment (start 92.885 48.895) (end 92.71 48.895) (width 1) (layer B.Cu) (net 3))
 (segment (start 92.71 48.895) (end 91.44 47.625) (width 1) (layer B.Cu) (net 3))
 (segment (start 91.44 47.625) (end 91.44 43.815) (width 1) (layer B.Cu) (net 3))
 (segment (start 80.645 33.02) (end 69.58 33.02) (width 1) (layer B.Cu) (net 3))
 (segment (start 66.04 36.195) (end 66.04 33.02) (width 1) (layer B.Cu) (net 3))
 (segment (start 66.04 33.02) (end 80.645 33.02) (width 1) (layer B.Cu) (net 3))
 (segment (start 58.42 33.02) (end 66.04 33.02) (width 1) (layer B.Cu) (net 3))
 (segment (start 89.535 135.255) (end 69.85 115.57) (width 1) (layer B.Cu) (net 3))
 (segment (start 69.85 115.57) (end 57.15 115.57) (width 1) (layer B.Cu) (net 3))
 (segment (start 57.15 115.57) (end 53.975 112.395) (width 1) (layer B.Cu) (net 3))
 (segment (start 53.975 112.395) (end 53.975 37.465) (width 1) (layer B.Cu) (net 3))
 (segment (start 53.975 37.465) (end 58.42 33.02) (width 1) (layer B.Cu) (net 3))
 (segment (start 67.31 43.18) (end 71.755 43.18) (width 1) (layer B.Cu) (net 3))
 (segment (start 66.04 42.545) (end 67.31 43.18) (width 1) (layer B.Cu) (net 3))
 (segment (start 105.87 53.34) (end 100.925 53.34) (width 1) (layer B.Cu) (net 3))
 (segment (start 113.665 45.545) (end 105.87 53.34) (width 1) (layer B.Cu) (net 3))
 (segment (start 113.665 42.545) (end 113.665 45.545) (width 1) (layer B.Cu) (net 3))
 (segment (start 83.82 36.195) (end 83.5025 35.8775) (width 1) (layer B.Cu) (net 3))
 (segment (start 113.665 36.195) (end 83.82 36.195) (width 1) (layer B.Cu) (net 3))
 (segment (start 91.44 43.815) (end 83.5025 35.8775) (width 1) (layer B.Cu) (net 3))
 (segment (start 83.5025 35.8775) (end 80.645 33.02) (width 1) (layer B.Cu) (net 3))
 (segment (start 109.22 148.59) (end 108.355823 148.59) (width 1) (layer B.Cu) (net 3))
 (segment (start 96.53 117.405) (end 95.805 116.68) (width 1) (layer B.Cu) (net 20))
 (segment (start 93.98 114.935) (end 93.98 110.49) (width 1) (layer B.Cu) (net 20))
 (segment (start 95.805 116.68) (end 95.725 116.68) (width 1) (layer B.Cu) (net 20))
 (segment (start 95.725 116.68) (end 93.98 114.935) (width 1) (layer B.Cu) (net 20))
 (segment (start 96.53 120.53) (end 96.53 117.405) (width 1) (layer B.Cu) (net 20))
 (segment (start 59.69 110.49) (end 64.77 110.49) (width 1) (layer B.Cu) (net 10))
 (segment (start 64.77 110.49) (end 71.12 110.49) (width 1) (layer B.Cu) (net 10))
 (segment (start 104.14 97.79) (end 104.14 102.87) (width 1) (layer B.Cu) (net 17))
 (segment (start 99.06 96.52) (end 99.06 102.87) (width 1) (layer B.Cu) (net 32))
 (segment (start 92.71 90.17) (end 99.06 96.52) (width 1) (layer B.Cu) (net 32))
 (segment (start 96.52 104.775) (end 96.52 102.87) (width 1) (layer B.Cu) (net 31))
 (segment (start 97.663 105.918) (end 96.52 104.775) (width 1) (layer B.Cu) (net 31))
 (segment (start 105.537 105.918) (end 97.663 105.918) (width 1) (layer B.Cu) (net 31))
 (segment (start 90.17 85.09) (end 92.71 82.55) (width 1) (layer B.Cu) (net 31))
 (segment (start 90.17 87.63) (end 90.17 85.09) (width 1) (layer B.Cu) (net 31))
 (segment (start 92.71 82.55) (end 95.25 82.55) (width 1) (layer B.Cu) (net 31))
 (segment (start 95.25 82.55) (end 107.315 94.615) (width 1) (layer B.Cu) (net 31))
 (segment (start 107.315 94.615) (end 107.315 104.14) (width 1) (layer B.Cu) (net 31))
 (segment (start 107.315 104.14) (end 105.537 105.918) (width 1) (layer B.Cu) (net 31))
 (segment (start 81.28 113.49) (end 81.28 110.49) (width 1) (layer B.Cu) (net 18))
 (segment (start 81.28 123.19) (end 81.28 113.49) (width 1) (layer B.Cu) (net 18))
 (segment (start 96.52 107.315) (end 93.98 104.775) (width 1) (layer B.Cu) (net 30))
 (segment (start 107.315 107.315) (end 96.52 107.315) (width 1) (layer B.Cu) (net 30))
 (segment (start 109.22 105.41) (end 107.315 107.315) (width 1) (layer B.Cu) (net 30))
 (segment (start 93.98 104.775) (end 93.98 102.87) (width 1) (layer B.Cu) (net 30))
 (segment (start 86.995 86.995) (end 86.995 84.455) (width 1) (layer B.Cu) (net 30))
 (segment (start 90.17 90.17) (end 86.995 86.995) (width 1) (layer B.Cu) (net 30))
 (segment (start 86.995 84.455) (end 90.17 81.28) (width 1) (layer B.Cu) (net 30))
 (segment (start 90.17 81.28) (end 99.695 81.28) (width 1) (layer B.Cu) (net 30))
 (segment (start 99.695 81.28) (end 109.22 90.805) (width 1) (layer B.Cu) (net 30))
 (segment (start 109.22 90.805) (end 109.22 105.41) (width 1) (layer B.Cu) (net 30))
 (segment (start 59.69 64.135) (end 59.69 69.85) (width 1) (layer B.Cu) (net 4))
 (segment (start 66.04 106.68) (end 59.69 100.33) (width 1) (layer B.Cu) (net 4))
 (segment (start 85.09 106.68) (end 66.04 106.68) (width 1) (layer B.Cu) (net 4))
 (segment (start 86.36 110.49) (end 86.36 107.95) (width 1) (layer B.Cu) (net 4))
 (segment (start 86.36 107.95) (end 85.09 106.68) (width 1) (layer B.Cu) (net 4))
 (segment (start 86.36 111.76) (end 86.36 110.49) (width 1) (layer B.Cu) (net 4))
 (segment (start 83.82 115.57) (end 83.82 114.3) (width 1) (layer B.Cu) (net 4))
 (segment (start 83.82 114.3) (end 86.36 111.76) (width 1) (layer B.Cu) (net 4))
 (segment (start 78.105 40.64) (end 79.375 41.91) (width 1) (layer B.Cu) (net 4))
 (segment (start 74.93 40.64) (end 78.105 40.64) (width 1) (layer B.Cu) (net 4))
 (segment (start 79.375 41.91) (end 79.375 44.45) (width 1) (layer B.Cu) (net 4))
 (segment (start 79.375 44.45) (end 62.865 60.96) (width 1) (layer B.Cu) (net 4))
 (segment (start 76.2 60.96) (end 67.485 60.96) (width 1) (layer B.Cu) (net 4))
 (segment (start 79.375 64.135) (end 76.2 60.96) (width 1) (layer B.Cu) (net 4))
 (segment (start 67.485 60.96) (end 62.865 60.96) (width 1) (layer B.Cu) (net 4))
 (segment (start 59.69 97.33) (end 59.69 64.135) (width 1) (layer B.Cu) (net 4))
 (segment (start 59.69 100.33) (end 59.69 97.33) (width 1) (layer B.Cu) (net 4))
 (segment (start 62.865 60.96) (end 59.69 64.135) (width 1) (layer B.Cu) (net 4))
 (segment (start 74.93 40.64) (end 71.755 40.64) (width 1) (layer B.Cu) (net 4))
 (segment (start 106.775 133.985) (end 104.775 133.985) (width 1) (layer B.Cu) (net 4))
 (segment (start 109.22 136.43) (end 106.775 133.985) (width 1) (layer B.Cu) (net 4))
 (segment (start 109.22 146.05) (end 109.22 136.43) (width 1) (layer B.Cu) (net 4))
 (segment (start 96.52 112.9425) (end 96.52 110.49) (width 1) (layer B.Cu) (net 7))
 (segment (start 107.9975 124.42) (end 96.52 112.9425) (width 1) (layer B.Cu) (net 7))
 (segment (start 99.06 110.49) (end 99.06 111.49) (width 1) (layer B.Cu) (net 8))
 (segment (start 99.06 112.395) (end 99.06 110.49) (width 1) (layer B.Cu) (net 8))
 (segment (start 106.085 119.42) (end 99.06 112.395) (width 1) (layer B.Cu) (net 8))
 (segment (start 73.66 99.695) (end 73.66 102.87) (width 1) (layer B.Cu) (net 15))
 (segment (start 86.36 55.88) (end 82.55 59.69) (width 1) (layer B.Cu) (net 15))
 (segment (start 86.36 53.34) (end 86.36 55.88) (width 1) (layer B.Cu) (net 15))
 (segment (start 82.55 59.69) (end 82.55 74.295) (width 1) (layer B.Cu) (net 15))
 (segment (start 82.55 74.295) (end 76.2 80.645) (width 1) (layer B.Cu) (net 15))
 (segment (start 76.2 80.645) (end 76.2 97.155) (width 1) (layer B.Cu) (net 15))
 (segment (start 76.2 97.155) (end 73.66 99.695) (width 1) (layer B.Cu) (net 15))
 (segment (start 74.93 38.1) (end 71.755 38.1) (width 1) (layer B.Cu) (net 15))
 (segment (start 78.74 38.1) (end 74.93 38.1) (width 1) (layer B.Cu) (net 15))
 (segment (start 86.36 53.34) (end 86.36 45.72) (width 1) (layer B.Cu) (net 15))
 (segment (start 86.36 45.72) (end 78.74 38.1) (width 1) (layer B.Cu) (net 15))
 (segment (start 71.12 102.87) (end 71.12 103.87) (width 1) (layer B.Cu) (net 14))
 (segment (start 71.12 86.36) (end 70.12 86.36) (width 1) (layer B.Cu) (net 14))
 (segment (start 71.12 86.36) (end 71.96293 86.36) (width 1) (layer B.Cu) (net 14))
 (segment (start 71.12 98.7425) (end 71.12 102.87) (width 1) (layer B.Cu) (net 14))
 (segment (start 74.295 95.5675) (end 71.12 98.7425) (width 1) (layer B.Cu) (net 14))
 (segment (start 71.12 86.36) (end 74.295 89.535) (width 1) (layer B.Cu) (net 14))
 (segment (start 74.295 89.535) (end 74.295 95.5675) (width 1) (layer B.Cu) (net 14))
 (segment (start 88.9 56.34) (end 88.9 53.34) (width 1) (layer B.Cu) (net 14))
 (segment (start 85.09 60.15) (end 88.9 56.34) (width 1) (layer B.Cu) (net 14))
 (segment (start 85.09 75.565) (end 85.09 60.15) (width 1) (layer B.Cu) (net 14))
 (segment (start 81.28 86.36) (end 81.28 79.375) (width 1) (layer B.Cu) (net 14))
 (segment (start 81.28 79.375) (end 85.09 75.565) (width 1) (layer B.Cu) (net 14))
 (segment (start 74.93 35.56) (end 71.755 35.56) (width 1) (layer B.Cu) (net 14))
 (segment (start 79.375 35.56) (end 74.93 35.56) (width 1) (layer B.Cu) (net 14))
 (segment (start 88.9 53.34) (end 88.9 45.085) (width 1) (layer B.Cu) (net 14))
 (segment (start 88.9 45.085) (end 79.375 35.56) (width 1) (layer B.Cu) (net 14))
 (segment (start 98.425 53.34) (end 93.98 53.34) (width 1) (layer B.Cu) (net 19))
 (segment (start 93.94 61.42) (end 93.94 58.42) (width 1) (layer B.Cu) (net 19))
 (segment (start 93.94 62.19) (end 93.94 61.42) (width 1) (layer B.Cu) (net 19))
 (segment (start 92.075 64.135) (end 93.98 62.23) (width 1) (layer B.Cu) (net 19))
 (segment (start 93.98 62.23) (end 93.94 62.19) (width 1) (layer B.Cu) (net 19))
 (segment (start 93.94 53.38) (end 93.98 53.34) (width 1) (layer B.Cu) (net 19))
 (segment (start 93.94 58.42) (end 93.94 53.38) (width 1) (layer B.Cu) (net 19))
 (segment (start 56.515 47.625) (end 61.595 42.545) (width 1) (layer B.Cu) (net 13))
 (segment (start 56.515 111.76) (end 56.515 47.625) (width 1) (layer B.Cu) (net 13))
 (segment (start 58.42 113.665) (end 56.515 111.76) (width 1) (layer B.Cu) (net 13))
 (segment (start 78.105 113.665) (end 58.42 113.665) (width 1) (layer B.Cu) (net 13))
 (segment (start 78.74 110.49) (end 78.74 113.03) (width 1) (layer B.Cu) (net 13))
 (segment (start 78.74 113.03) (end 78.105 113.665) (width 1) (layer B.Cu) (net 13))
 (segment (start 107.95 110.49) (end 104.14 110.49) (width 1) (layer B.Cu) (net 12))
 (segment (start 111.125 107.315) (end 107.95 110.49) (width 1) (layer B.Cu) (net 12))
 (segment (start 118.11 47.625) (end 118.11 42.545) (width 1) (layer B.Cu) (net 12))
 (segment (start 111.125 54.61) (end 118.11 47.625) (width 1) (layer B.Cu) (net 12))
 (segment (start 111.125 54.61) (end 111.125 107.315) (width 1) (layer B.Cu) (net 12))
 (segment (start 108.355823 151.13) (end 109.22 151.13) (width 1) (layer B.Cu) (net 2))
 (segment (start 100.965 140.065) (end 102.505 141.605) (width 1) (layer B.Cu) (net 2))
 (segment (start 100.965 139.065) (end 100.965 140.065) (width 1) (layer B.Cu) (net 2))
 (segment (start 102.505 141.605) (end 103.630318 141.605) (width 1) (layer B.Cu) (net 2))
 (segment (start 103.630318 141.605) (end 105.41 143.384682) (width 1) (layer B.Cu) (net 2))
 (segment (start 105.41 143.384682) (end 105.41 148.184177) (width 1) (layer B.Cu) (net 2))
 (segment (start 105.41 148.184177) (end 108.355823 151.13) (width 1) (layer B.Cu) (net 2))
 (segment (start 109.22 153.835) (end 112.395 157.01) (width 1) (layer B.Cu) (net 2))
 (segment (start 109.22 151.13) (end 109.22 153.835) (width 1) (layer B.Cu) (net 2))
 (segment (start 114.3 136.59) (end 116.15 134.74) (width 1) (layer B.Cu) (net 2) (status 1000000))
 (segment (start 112.395 157.01) (end 114.3 155.105) (width 1) (layer B.Cu) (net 2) (status 1000000))
 (segment (start 114.3 155.105) (end 114.3 136.59) (width 1) (layer B.Cu) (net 2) (status 1000000))
 (segment (start 116.15 134.74) (end 117.15 134.74) (width 1) (layer B.Cu) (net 2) (status 1000000))
 (segment (start 117.15 179.255) (end 114.395 182.01) (width 1) (layer B.Cu) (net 1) (status 1000000))
 (segment (start 114.395 182.01) (end 112.395 182.01) (width 1) (layer B.Cu) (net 1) (status 1000000))
 (segment (start 117.15 149.74) (end 117.15 179.255) (width 1) (layer B.Cu) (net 1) (status 1000000))
 (segment (start 117.15 144.74) (end 117.15 139.74) (width 1) (layer B.Cu) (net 5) (status 1000000))
 (segment (start 114.3 107.95) (end 114.3 97.79) (width 1) (layer B.Cu) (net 9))
 (segment (start 64.77 99.695) (end 71.12 93.345) (width 1) (layer B.Cu) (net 11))
 (segment (start 64.77 100.33) (end 64.77 99.695) (width 1) (layer B.Cu) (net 11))
 (segment (start 89.535 93.345) (end 90.17 92.71) (width 1) (layer B.Cu) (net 16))
 (segment (start 81.28 93.345) (end 89.535 93.345) (width 1) (layer B.Cu) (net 16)))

